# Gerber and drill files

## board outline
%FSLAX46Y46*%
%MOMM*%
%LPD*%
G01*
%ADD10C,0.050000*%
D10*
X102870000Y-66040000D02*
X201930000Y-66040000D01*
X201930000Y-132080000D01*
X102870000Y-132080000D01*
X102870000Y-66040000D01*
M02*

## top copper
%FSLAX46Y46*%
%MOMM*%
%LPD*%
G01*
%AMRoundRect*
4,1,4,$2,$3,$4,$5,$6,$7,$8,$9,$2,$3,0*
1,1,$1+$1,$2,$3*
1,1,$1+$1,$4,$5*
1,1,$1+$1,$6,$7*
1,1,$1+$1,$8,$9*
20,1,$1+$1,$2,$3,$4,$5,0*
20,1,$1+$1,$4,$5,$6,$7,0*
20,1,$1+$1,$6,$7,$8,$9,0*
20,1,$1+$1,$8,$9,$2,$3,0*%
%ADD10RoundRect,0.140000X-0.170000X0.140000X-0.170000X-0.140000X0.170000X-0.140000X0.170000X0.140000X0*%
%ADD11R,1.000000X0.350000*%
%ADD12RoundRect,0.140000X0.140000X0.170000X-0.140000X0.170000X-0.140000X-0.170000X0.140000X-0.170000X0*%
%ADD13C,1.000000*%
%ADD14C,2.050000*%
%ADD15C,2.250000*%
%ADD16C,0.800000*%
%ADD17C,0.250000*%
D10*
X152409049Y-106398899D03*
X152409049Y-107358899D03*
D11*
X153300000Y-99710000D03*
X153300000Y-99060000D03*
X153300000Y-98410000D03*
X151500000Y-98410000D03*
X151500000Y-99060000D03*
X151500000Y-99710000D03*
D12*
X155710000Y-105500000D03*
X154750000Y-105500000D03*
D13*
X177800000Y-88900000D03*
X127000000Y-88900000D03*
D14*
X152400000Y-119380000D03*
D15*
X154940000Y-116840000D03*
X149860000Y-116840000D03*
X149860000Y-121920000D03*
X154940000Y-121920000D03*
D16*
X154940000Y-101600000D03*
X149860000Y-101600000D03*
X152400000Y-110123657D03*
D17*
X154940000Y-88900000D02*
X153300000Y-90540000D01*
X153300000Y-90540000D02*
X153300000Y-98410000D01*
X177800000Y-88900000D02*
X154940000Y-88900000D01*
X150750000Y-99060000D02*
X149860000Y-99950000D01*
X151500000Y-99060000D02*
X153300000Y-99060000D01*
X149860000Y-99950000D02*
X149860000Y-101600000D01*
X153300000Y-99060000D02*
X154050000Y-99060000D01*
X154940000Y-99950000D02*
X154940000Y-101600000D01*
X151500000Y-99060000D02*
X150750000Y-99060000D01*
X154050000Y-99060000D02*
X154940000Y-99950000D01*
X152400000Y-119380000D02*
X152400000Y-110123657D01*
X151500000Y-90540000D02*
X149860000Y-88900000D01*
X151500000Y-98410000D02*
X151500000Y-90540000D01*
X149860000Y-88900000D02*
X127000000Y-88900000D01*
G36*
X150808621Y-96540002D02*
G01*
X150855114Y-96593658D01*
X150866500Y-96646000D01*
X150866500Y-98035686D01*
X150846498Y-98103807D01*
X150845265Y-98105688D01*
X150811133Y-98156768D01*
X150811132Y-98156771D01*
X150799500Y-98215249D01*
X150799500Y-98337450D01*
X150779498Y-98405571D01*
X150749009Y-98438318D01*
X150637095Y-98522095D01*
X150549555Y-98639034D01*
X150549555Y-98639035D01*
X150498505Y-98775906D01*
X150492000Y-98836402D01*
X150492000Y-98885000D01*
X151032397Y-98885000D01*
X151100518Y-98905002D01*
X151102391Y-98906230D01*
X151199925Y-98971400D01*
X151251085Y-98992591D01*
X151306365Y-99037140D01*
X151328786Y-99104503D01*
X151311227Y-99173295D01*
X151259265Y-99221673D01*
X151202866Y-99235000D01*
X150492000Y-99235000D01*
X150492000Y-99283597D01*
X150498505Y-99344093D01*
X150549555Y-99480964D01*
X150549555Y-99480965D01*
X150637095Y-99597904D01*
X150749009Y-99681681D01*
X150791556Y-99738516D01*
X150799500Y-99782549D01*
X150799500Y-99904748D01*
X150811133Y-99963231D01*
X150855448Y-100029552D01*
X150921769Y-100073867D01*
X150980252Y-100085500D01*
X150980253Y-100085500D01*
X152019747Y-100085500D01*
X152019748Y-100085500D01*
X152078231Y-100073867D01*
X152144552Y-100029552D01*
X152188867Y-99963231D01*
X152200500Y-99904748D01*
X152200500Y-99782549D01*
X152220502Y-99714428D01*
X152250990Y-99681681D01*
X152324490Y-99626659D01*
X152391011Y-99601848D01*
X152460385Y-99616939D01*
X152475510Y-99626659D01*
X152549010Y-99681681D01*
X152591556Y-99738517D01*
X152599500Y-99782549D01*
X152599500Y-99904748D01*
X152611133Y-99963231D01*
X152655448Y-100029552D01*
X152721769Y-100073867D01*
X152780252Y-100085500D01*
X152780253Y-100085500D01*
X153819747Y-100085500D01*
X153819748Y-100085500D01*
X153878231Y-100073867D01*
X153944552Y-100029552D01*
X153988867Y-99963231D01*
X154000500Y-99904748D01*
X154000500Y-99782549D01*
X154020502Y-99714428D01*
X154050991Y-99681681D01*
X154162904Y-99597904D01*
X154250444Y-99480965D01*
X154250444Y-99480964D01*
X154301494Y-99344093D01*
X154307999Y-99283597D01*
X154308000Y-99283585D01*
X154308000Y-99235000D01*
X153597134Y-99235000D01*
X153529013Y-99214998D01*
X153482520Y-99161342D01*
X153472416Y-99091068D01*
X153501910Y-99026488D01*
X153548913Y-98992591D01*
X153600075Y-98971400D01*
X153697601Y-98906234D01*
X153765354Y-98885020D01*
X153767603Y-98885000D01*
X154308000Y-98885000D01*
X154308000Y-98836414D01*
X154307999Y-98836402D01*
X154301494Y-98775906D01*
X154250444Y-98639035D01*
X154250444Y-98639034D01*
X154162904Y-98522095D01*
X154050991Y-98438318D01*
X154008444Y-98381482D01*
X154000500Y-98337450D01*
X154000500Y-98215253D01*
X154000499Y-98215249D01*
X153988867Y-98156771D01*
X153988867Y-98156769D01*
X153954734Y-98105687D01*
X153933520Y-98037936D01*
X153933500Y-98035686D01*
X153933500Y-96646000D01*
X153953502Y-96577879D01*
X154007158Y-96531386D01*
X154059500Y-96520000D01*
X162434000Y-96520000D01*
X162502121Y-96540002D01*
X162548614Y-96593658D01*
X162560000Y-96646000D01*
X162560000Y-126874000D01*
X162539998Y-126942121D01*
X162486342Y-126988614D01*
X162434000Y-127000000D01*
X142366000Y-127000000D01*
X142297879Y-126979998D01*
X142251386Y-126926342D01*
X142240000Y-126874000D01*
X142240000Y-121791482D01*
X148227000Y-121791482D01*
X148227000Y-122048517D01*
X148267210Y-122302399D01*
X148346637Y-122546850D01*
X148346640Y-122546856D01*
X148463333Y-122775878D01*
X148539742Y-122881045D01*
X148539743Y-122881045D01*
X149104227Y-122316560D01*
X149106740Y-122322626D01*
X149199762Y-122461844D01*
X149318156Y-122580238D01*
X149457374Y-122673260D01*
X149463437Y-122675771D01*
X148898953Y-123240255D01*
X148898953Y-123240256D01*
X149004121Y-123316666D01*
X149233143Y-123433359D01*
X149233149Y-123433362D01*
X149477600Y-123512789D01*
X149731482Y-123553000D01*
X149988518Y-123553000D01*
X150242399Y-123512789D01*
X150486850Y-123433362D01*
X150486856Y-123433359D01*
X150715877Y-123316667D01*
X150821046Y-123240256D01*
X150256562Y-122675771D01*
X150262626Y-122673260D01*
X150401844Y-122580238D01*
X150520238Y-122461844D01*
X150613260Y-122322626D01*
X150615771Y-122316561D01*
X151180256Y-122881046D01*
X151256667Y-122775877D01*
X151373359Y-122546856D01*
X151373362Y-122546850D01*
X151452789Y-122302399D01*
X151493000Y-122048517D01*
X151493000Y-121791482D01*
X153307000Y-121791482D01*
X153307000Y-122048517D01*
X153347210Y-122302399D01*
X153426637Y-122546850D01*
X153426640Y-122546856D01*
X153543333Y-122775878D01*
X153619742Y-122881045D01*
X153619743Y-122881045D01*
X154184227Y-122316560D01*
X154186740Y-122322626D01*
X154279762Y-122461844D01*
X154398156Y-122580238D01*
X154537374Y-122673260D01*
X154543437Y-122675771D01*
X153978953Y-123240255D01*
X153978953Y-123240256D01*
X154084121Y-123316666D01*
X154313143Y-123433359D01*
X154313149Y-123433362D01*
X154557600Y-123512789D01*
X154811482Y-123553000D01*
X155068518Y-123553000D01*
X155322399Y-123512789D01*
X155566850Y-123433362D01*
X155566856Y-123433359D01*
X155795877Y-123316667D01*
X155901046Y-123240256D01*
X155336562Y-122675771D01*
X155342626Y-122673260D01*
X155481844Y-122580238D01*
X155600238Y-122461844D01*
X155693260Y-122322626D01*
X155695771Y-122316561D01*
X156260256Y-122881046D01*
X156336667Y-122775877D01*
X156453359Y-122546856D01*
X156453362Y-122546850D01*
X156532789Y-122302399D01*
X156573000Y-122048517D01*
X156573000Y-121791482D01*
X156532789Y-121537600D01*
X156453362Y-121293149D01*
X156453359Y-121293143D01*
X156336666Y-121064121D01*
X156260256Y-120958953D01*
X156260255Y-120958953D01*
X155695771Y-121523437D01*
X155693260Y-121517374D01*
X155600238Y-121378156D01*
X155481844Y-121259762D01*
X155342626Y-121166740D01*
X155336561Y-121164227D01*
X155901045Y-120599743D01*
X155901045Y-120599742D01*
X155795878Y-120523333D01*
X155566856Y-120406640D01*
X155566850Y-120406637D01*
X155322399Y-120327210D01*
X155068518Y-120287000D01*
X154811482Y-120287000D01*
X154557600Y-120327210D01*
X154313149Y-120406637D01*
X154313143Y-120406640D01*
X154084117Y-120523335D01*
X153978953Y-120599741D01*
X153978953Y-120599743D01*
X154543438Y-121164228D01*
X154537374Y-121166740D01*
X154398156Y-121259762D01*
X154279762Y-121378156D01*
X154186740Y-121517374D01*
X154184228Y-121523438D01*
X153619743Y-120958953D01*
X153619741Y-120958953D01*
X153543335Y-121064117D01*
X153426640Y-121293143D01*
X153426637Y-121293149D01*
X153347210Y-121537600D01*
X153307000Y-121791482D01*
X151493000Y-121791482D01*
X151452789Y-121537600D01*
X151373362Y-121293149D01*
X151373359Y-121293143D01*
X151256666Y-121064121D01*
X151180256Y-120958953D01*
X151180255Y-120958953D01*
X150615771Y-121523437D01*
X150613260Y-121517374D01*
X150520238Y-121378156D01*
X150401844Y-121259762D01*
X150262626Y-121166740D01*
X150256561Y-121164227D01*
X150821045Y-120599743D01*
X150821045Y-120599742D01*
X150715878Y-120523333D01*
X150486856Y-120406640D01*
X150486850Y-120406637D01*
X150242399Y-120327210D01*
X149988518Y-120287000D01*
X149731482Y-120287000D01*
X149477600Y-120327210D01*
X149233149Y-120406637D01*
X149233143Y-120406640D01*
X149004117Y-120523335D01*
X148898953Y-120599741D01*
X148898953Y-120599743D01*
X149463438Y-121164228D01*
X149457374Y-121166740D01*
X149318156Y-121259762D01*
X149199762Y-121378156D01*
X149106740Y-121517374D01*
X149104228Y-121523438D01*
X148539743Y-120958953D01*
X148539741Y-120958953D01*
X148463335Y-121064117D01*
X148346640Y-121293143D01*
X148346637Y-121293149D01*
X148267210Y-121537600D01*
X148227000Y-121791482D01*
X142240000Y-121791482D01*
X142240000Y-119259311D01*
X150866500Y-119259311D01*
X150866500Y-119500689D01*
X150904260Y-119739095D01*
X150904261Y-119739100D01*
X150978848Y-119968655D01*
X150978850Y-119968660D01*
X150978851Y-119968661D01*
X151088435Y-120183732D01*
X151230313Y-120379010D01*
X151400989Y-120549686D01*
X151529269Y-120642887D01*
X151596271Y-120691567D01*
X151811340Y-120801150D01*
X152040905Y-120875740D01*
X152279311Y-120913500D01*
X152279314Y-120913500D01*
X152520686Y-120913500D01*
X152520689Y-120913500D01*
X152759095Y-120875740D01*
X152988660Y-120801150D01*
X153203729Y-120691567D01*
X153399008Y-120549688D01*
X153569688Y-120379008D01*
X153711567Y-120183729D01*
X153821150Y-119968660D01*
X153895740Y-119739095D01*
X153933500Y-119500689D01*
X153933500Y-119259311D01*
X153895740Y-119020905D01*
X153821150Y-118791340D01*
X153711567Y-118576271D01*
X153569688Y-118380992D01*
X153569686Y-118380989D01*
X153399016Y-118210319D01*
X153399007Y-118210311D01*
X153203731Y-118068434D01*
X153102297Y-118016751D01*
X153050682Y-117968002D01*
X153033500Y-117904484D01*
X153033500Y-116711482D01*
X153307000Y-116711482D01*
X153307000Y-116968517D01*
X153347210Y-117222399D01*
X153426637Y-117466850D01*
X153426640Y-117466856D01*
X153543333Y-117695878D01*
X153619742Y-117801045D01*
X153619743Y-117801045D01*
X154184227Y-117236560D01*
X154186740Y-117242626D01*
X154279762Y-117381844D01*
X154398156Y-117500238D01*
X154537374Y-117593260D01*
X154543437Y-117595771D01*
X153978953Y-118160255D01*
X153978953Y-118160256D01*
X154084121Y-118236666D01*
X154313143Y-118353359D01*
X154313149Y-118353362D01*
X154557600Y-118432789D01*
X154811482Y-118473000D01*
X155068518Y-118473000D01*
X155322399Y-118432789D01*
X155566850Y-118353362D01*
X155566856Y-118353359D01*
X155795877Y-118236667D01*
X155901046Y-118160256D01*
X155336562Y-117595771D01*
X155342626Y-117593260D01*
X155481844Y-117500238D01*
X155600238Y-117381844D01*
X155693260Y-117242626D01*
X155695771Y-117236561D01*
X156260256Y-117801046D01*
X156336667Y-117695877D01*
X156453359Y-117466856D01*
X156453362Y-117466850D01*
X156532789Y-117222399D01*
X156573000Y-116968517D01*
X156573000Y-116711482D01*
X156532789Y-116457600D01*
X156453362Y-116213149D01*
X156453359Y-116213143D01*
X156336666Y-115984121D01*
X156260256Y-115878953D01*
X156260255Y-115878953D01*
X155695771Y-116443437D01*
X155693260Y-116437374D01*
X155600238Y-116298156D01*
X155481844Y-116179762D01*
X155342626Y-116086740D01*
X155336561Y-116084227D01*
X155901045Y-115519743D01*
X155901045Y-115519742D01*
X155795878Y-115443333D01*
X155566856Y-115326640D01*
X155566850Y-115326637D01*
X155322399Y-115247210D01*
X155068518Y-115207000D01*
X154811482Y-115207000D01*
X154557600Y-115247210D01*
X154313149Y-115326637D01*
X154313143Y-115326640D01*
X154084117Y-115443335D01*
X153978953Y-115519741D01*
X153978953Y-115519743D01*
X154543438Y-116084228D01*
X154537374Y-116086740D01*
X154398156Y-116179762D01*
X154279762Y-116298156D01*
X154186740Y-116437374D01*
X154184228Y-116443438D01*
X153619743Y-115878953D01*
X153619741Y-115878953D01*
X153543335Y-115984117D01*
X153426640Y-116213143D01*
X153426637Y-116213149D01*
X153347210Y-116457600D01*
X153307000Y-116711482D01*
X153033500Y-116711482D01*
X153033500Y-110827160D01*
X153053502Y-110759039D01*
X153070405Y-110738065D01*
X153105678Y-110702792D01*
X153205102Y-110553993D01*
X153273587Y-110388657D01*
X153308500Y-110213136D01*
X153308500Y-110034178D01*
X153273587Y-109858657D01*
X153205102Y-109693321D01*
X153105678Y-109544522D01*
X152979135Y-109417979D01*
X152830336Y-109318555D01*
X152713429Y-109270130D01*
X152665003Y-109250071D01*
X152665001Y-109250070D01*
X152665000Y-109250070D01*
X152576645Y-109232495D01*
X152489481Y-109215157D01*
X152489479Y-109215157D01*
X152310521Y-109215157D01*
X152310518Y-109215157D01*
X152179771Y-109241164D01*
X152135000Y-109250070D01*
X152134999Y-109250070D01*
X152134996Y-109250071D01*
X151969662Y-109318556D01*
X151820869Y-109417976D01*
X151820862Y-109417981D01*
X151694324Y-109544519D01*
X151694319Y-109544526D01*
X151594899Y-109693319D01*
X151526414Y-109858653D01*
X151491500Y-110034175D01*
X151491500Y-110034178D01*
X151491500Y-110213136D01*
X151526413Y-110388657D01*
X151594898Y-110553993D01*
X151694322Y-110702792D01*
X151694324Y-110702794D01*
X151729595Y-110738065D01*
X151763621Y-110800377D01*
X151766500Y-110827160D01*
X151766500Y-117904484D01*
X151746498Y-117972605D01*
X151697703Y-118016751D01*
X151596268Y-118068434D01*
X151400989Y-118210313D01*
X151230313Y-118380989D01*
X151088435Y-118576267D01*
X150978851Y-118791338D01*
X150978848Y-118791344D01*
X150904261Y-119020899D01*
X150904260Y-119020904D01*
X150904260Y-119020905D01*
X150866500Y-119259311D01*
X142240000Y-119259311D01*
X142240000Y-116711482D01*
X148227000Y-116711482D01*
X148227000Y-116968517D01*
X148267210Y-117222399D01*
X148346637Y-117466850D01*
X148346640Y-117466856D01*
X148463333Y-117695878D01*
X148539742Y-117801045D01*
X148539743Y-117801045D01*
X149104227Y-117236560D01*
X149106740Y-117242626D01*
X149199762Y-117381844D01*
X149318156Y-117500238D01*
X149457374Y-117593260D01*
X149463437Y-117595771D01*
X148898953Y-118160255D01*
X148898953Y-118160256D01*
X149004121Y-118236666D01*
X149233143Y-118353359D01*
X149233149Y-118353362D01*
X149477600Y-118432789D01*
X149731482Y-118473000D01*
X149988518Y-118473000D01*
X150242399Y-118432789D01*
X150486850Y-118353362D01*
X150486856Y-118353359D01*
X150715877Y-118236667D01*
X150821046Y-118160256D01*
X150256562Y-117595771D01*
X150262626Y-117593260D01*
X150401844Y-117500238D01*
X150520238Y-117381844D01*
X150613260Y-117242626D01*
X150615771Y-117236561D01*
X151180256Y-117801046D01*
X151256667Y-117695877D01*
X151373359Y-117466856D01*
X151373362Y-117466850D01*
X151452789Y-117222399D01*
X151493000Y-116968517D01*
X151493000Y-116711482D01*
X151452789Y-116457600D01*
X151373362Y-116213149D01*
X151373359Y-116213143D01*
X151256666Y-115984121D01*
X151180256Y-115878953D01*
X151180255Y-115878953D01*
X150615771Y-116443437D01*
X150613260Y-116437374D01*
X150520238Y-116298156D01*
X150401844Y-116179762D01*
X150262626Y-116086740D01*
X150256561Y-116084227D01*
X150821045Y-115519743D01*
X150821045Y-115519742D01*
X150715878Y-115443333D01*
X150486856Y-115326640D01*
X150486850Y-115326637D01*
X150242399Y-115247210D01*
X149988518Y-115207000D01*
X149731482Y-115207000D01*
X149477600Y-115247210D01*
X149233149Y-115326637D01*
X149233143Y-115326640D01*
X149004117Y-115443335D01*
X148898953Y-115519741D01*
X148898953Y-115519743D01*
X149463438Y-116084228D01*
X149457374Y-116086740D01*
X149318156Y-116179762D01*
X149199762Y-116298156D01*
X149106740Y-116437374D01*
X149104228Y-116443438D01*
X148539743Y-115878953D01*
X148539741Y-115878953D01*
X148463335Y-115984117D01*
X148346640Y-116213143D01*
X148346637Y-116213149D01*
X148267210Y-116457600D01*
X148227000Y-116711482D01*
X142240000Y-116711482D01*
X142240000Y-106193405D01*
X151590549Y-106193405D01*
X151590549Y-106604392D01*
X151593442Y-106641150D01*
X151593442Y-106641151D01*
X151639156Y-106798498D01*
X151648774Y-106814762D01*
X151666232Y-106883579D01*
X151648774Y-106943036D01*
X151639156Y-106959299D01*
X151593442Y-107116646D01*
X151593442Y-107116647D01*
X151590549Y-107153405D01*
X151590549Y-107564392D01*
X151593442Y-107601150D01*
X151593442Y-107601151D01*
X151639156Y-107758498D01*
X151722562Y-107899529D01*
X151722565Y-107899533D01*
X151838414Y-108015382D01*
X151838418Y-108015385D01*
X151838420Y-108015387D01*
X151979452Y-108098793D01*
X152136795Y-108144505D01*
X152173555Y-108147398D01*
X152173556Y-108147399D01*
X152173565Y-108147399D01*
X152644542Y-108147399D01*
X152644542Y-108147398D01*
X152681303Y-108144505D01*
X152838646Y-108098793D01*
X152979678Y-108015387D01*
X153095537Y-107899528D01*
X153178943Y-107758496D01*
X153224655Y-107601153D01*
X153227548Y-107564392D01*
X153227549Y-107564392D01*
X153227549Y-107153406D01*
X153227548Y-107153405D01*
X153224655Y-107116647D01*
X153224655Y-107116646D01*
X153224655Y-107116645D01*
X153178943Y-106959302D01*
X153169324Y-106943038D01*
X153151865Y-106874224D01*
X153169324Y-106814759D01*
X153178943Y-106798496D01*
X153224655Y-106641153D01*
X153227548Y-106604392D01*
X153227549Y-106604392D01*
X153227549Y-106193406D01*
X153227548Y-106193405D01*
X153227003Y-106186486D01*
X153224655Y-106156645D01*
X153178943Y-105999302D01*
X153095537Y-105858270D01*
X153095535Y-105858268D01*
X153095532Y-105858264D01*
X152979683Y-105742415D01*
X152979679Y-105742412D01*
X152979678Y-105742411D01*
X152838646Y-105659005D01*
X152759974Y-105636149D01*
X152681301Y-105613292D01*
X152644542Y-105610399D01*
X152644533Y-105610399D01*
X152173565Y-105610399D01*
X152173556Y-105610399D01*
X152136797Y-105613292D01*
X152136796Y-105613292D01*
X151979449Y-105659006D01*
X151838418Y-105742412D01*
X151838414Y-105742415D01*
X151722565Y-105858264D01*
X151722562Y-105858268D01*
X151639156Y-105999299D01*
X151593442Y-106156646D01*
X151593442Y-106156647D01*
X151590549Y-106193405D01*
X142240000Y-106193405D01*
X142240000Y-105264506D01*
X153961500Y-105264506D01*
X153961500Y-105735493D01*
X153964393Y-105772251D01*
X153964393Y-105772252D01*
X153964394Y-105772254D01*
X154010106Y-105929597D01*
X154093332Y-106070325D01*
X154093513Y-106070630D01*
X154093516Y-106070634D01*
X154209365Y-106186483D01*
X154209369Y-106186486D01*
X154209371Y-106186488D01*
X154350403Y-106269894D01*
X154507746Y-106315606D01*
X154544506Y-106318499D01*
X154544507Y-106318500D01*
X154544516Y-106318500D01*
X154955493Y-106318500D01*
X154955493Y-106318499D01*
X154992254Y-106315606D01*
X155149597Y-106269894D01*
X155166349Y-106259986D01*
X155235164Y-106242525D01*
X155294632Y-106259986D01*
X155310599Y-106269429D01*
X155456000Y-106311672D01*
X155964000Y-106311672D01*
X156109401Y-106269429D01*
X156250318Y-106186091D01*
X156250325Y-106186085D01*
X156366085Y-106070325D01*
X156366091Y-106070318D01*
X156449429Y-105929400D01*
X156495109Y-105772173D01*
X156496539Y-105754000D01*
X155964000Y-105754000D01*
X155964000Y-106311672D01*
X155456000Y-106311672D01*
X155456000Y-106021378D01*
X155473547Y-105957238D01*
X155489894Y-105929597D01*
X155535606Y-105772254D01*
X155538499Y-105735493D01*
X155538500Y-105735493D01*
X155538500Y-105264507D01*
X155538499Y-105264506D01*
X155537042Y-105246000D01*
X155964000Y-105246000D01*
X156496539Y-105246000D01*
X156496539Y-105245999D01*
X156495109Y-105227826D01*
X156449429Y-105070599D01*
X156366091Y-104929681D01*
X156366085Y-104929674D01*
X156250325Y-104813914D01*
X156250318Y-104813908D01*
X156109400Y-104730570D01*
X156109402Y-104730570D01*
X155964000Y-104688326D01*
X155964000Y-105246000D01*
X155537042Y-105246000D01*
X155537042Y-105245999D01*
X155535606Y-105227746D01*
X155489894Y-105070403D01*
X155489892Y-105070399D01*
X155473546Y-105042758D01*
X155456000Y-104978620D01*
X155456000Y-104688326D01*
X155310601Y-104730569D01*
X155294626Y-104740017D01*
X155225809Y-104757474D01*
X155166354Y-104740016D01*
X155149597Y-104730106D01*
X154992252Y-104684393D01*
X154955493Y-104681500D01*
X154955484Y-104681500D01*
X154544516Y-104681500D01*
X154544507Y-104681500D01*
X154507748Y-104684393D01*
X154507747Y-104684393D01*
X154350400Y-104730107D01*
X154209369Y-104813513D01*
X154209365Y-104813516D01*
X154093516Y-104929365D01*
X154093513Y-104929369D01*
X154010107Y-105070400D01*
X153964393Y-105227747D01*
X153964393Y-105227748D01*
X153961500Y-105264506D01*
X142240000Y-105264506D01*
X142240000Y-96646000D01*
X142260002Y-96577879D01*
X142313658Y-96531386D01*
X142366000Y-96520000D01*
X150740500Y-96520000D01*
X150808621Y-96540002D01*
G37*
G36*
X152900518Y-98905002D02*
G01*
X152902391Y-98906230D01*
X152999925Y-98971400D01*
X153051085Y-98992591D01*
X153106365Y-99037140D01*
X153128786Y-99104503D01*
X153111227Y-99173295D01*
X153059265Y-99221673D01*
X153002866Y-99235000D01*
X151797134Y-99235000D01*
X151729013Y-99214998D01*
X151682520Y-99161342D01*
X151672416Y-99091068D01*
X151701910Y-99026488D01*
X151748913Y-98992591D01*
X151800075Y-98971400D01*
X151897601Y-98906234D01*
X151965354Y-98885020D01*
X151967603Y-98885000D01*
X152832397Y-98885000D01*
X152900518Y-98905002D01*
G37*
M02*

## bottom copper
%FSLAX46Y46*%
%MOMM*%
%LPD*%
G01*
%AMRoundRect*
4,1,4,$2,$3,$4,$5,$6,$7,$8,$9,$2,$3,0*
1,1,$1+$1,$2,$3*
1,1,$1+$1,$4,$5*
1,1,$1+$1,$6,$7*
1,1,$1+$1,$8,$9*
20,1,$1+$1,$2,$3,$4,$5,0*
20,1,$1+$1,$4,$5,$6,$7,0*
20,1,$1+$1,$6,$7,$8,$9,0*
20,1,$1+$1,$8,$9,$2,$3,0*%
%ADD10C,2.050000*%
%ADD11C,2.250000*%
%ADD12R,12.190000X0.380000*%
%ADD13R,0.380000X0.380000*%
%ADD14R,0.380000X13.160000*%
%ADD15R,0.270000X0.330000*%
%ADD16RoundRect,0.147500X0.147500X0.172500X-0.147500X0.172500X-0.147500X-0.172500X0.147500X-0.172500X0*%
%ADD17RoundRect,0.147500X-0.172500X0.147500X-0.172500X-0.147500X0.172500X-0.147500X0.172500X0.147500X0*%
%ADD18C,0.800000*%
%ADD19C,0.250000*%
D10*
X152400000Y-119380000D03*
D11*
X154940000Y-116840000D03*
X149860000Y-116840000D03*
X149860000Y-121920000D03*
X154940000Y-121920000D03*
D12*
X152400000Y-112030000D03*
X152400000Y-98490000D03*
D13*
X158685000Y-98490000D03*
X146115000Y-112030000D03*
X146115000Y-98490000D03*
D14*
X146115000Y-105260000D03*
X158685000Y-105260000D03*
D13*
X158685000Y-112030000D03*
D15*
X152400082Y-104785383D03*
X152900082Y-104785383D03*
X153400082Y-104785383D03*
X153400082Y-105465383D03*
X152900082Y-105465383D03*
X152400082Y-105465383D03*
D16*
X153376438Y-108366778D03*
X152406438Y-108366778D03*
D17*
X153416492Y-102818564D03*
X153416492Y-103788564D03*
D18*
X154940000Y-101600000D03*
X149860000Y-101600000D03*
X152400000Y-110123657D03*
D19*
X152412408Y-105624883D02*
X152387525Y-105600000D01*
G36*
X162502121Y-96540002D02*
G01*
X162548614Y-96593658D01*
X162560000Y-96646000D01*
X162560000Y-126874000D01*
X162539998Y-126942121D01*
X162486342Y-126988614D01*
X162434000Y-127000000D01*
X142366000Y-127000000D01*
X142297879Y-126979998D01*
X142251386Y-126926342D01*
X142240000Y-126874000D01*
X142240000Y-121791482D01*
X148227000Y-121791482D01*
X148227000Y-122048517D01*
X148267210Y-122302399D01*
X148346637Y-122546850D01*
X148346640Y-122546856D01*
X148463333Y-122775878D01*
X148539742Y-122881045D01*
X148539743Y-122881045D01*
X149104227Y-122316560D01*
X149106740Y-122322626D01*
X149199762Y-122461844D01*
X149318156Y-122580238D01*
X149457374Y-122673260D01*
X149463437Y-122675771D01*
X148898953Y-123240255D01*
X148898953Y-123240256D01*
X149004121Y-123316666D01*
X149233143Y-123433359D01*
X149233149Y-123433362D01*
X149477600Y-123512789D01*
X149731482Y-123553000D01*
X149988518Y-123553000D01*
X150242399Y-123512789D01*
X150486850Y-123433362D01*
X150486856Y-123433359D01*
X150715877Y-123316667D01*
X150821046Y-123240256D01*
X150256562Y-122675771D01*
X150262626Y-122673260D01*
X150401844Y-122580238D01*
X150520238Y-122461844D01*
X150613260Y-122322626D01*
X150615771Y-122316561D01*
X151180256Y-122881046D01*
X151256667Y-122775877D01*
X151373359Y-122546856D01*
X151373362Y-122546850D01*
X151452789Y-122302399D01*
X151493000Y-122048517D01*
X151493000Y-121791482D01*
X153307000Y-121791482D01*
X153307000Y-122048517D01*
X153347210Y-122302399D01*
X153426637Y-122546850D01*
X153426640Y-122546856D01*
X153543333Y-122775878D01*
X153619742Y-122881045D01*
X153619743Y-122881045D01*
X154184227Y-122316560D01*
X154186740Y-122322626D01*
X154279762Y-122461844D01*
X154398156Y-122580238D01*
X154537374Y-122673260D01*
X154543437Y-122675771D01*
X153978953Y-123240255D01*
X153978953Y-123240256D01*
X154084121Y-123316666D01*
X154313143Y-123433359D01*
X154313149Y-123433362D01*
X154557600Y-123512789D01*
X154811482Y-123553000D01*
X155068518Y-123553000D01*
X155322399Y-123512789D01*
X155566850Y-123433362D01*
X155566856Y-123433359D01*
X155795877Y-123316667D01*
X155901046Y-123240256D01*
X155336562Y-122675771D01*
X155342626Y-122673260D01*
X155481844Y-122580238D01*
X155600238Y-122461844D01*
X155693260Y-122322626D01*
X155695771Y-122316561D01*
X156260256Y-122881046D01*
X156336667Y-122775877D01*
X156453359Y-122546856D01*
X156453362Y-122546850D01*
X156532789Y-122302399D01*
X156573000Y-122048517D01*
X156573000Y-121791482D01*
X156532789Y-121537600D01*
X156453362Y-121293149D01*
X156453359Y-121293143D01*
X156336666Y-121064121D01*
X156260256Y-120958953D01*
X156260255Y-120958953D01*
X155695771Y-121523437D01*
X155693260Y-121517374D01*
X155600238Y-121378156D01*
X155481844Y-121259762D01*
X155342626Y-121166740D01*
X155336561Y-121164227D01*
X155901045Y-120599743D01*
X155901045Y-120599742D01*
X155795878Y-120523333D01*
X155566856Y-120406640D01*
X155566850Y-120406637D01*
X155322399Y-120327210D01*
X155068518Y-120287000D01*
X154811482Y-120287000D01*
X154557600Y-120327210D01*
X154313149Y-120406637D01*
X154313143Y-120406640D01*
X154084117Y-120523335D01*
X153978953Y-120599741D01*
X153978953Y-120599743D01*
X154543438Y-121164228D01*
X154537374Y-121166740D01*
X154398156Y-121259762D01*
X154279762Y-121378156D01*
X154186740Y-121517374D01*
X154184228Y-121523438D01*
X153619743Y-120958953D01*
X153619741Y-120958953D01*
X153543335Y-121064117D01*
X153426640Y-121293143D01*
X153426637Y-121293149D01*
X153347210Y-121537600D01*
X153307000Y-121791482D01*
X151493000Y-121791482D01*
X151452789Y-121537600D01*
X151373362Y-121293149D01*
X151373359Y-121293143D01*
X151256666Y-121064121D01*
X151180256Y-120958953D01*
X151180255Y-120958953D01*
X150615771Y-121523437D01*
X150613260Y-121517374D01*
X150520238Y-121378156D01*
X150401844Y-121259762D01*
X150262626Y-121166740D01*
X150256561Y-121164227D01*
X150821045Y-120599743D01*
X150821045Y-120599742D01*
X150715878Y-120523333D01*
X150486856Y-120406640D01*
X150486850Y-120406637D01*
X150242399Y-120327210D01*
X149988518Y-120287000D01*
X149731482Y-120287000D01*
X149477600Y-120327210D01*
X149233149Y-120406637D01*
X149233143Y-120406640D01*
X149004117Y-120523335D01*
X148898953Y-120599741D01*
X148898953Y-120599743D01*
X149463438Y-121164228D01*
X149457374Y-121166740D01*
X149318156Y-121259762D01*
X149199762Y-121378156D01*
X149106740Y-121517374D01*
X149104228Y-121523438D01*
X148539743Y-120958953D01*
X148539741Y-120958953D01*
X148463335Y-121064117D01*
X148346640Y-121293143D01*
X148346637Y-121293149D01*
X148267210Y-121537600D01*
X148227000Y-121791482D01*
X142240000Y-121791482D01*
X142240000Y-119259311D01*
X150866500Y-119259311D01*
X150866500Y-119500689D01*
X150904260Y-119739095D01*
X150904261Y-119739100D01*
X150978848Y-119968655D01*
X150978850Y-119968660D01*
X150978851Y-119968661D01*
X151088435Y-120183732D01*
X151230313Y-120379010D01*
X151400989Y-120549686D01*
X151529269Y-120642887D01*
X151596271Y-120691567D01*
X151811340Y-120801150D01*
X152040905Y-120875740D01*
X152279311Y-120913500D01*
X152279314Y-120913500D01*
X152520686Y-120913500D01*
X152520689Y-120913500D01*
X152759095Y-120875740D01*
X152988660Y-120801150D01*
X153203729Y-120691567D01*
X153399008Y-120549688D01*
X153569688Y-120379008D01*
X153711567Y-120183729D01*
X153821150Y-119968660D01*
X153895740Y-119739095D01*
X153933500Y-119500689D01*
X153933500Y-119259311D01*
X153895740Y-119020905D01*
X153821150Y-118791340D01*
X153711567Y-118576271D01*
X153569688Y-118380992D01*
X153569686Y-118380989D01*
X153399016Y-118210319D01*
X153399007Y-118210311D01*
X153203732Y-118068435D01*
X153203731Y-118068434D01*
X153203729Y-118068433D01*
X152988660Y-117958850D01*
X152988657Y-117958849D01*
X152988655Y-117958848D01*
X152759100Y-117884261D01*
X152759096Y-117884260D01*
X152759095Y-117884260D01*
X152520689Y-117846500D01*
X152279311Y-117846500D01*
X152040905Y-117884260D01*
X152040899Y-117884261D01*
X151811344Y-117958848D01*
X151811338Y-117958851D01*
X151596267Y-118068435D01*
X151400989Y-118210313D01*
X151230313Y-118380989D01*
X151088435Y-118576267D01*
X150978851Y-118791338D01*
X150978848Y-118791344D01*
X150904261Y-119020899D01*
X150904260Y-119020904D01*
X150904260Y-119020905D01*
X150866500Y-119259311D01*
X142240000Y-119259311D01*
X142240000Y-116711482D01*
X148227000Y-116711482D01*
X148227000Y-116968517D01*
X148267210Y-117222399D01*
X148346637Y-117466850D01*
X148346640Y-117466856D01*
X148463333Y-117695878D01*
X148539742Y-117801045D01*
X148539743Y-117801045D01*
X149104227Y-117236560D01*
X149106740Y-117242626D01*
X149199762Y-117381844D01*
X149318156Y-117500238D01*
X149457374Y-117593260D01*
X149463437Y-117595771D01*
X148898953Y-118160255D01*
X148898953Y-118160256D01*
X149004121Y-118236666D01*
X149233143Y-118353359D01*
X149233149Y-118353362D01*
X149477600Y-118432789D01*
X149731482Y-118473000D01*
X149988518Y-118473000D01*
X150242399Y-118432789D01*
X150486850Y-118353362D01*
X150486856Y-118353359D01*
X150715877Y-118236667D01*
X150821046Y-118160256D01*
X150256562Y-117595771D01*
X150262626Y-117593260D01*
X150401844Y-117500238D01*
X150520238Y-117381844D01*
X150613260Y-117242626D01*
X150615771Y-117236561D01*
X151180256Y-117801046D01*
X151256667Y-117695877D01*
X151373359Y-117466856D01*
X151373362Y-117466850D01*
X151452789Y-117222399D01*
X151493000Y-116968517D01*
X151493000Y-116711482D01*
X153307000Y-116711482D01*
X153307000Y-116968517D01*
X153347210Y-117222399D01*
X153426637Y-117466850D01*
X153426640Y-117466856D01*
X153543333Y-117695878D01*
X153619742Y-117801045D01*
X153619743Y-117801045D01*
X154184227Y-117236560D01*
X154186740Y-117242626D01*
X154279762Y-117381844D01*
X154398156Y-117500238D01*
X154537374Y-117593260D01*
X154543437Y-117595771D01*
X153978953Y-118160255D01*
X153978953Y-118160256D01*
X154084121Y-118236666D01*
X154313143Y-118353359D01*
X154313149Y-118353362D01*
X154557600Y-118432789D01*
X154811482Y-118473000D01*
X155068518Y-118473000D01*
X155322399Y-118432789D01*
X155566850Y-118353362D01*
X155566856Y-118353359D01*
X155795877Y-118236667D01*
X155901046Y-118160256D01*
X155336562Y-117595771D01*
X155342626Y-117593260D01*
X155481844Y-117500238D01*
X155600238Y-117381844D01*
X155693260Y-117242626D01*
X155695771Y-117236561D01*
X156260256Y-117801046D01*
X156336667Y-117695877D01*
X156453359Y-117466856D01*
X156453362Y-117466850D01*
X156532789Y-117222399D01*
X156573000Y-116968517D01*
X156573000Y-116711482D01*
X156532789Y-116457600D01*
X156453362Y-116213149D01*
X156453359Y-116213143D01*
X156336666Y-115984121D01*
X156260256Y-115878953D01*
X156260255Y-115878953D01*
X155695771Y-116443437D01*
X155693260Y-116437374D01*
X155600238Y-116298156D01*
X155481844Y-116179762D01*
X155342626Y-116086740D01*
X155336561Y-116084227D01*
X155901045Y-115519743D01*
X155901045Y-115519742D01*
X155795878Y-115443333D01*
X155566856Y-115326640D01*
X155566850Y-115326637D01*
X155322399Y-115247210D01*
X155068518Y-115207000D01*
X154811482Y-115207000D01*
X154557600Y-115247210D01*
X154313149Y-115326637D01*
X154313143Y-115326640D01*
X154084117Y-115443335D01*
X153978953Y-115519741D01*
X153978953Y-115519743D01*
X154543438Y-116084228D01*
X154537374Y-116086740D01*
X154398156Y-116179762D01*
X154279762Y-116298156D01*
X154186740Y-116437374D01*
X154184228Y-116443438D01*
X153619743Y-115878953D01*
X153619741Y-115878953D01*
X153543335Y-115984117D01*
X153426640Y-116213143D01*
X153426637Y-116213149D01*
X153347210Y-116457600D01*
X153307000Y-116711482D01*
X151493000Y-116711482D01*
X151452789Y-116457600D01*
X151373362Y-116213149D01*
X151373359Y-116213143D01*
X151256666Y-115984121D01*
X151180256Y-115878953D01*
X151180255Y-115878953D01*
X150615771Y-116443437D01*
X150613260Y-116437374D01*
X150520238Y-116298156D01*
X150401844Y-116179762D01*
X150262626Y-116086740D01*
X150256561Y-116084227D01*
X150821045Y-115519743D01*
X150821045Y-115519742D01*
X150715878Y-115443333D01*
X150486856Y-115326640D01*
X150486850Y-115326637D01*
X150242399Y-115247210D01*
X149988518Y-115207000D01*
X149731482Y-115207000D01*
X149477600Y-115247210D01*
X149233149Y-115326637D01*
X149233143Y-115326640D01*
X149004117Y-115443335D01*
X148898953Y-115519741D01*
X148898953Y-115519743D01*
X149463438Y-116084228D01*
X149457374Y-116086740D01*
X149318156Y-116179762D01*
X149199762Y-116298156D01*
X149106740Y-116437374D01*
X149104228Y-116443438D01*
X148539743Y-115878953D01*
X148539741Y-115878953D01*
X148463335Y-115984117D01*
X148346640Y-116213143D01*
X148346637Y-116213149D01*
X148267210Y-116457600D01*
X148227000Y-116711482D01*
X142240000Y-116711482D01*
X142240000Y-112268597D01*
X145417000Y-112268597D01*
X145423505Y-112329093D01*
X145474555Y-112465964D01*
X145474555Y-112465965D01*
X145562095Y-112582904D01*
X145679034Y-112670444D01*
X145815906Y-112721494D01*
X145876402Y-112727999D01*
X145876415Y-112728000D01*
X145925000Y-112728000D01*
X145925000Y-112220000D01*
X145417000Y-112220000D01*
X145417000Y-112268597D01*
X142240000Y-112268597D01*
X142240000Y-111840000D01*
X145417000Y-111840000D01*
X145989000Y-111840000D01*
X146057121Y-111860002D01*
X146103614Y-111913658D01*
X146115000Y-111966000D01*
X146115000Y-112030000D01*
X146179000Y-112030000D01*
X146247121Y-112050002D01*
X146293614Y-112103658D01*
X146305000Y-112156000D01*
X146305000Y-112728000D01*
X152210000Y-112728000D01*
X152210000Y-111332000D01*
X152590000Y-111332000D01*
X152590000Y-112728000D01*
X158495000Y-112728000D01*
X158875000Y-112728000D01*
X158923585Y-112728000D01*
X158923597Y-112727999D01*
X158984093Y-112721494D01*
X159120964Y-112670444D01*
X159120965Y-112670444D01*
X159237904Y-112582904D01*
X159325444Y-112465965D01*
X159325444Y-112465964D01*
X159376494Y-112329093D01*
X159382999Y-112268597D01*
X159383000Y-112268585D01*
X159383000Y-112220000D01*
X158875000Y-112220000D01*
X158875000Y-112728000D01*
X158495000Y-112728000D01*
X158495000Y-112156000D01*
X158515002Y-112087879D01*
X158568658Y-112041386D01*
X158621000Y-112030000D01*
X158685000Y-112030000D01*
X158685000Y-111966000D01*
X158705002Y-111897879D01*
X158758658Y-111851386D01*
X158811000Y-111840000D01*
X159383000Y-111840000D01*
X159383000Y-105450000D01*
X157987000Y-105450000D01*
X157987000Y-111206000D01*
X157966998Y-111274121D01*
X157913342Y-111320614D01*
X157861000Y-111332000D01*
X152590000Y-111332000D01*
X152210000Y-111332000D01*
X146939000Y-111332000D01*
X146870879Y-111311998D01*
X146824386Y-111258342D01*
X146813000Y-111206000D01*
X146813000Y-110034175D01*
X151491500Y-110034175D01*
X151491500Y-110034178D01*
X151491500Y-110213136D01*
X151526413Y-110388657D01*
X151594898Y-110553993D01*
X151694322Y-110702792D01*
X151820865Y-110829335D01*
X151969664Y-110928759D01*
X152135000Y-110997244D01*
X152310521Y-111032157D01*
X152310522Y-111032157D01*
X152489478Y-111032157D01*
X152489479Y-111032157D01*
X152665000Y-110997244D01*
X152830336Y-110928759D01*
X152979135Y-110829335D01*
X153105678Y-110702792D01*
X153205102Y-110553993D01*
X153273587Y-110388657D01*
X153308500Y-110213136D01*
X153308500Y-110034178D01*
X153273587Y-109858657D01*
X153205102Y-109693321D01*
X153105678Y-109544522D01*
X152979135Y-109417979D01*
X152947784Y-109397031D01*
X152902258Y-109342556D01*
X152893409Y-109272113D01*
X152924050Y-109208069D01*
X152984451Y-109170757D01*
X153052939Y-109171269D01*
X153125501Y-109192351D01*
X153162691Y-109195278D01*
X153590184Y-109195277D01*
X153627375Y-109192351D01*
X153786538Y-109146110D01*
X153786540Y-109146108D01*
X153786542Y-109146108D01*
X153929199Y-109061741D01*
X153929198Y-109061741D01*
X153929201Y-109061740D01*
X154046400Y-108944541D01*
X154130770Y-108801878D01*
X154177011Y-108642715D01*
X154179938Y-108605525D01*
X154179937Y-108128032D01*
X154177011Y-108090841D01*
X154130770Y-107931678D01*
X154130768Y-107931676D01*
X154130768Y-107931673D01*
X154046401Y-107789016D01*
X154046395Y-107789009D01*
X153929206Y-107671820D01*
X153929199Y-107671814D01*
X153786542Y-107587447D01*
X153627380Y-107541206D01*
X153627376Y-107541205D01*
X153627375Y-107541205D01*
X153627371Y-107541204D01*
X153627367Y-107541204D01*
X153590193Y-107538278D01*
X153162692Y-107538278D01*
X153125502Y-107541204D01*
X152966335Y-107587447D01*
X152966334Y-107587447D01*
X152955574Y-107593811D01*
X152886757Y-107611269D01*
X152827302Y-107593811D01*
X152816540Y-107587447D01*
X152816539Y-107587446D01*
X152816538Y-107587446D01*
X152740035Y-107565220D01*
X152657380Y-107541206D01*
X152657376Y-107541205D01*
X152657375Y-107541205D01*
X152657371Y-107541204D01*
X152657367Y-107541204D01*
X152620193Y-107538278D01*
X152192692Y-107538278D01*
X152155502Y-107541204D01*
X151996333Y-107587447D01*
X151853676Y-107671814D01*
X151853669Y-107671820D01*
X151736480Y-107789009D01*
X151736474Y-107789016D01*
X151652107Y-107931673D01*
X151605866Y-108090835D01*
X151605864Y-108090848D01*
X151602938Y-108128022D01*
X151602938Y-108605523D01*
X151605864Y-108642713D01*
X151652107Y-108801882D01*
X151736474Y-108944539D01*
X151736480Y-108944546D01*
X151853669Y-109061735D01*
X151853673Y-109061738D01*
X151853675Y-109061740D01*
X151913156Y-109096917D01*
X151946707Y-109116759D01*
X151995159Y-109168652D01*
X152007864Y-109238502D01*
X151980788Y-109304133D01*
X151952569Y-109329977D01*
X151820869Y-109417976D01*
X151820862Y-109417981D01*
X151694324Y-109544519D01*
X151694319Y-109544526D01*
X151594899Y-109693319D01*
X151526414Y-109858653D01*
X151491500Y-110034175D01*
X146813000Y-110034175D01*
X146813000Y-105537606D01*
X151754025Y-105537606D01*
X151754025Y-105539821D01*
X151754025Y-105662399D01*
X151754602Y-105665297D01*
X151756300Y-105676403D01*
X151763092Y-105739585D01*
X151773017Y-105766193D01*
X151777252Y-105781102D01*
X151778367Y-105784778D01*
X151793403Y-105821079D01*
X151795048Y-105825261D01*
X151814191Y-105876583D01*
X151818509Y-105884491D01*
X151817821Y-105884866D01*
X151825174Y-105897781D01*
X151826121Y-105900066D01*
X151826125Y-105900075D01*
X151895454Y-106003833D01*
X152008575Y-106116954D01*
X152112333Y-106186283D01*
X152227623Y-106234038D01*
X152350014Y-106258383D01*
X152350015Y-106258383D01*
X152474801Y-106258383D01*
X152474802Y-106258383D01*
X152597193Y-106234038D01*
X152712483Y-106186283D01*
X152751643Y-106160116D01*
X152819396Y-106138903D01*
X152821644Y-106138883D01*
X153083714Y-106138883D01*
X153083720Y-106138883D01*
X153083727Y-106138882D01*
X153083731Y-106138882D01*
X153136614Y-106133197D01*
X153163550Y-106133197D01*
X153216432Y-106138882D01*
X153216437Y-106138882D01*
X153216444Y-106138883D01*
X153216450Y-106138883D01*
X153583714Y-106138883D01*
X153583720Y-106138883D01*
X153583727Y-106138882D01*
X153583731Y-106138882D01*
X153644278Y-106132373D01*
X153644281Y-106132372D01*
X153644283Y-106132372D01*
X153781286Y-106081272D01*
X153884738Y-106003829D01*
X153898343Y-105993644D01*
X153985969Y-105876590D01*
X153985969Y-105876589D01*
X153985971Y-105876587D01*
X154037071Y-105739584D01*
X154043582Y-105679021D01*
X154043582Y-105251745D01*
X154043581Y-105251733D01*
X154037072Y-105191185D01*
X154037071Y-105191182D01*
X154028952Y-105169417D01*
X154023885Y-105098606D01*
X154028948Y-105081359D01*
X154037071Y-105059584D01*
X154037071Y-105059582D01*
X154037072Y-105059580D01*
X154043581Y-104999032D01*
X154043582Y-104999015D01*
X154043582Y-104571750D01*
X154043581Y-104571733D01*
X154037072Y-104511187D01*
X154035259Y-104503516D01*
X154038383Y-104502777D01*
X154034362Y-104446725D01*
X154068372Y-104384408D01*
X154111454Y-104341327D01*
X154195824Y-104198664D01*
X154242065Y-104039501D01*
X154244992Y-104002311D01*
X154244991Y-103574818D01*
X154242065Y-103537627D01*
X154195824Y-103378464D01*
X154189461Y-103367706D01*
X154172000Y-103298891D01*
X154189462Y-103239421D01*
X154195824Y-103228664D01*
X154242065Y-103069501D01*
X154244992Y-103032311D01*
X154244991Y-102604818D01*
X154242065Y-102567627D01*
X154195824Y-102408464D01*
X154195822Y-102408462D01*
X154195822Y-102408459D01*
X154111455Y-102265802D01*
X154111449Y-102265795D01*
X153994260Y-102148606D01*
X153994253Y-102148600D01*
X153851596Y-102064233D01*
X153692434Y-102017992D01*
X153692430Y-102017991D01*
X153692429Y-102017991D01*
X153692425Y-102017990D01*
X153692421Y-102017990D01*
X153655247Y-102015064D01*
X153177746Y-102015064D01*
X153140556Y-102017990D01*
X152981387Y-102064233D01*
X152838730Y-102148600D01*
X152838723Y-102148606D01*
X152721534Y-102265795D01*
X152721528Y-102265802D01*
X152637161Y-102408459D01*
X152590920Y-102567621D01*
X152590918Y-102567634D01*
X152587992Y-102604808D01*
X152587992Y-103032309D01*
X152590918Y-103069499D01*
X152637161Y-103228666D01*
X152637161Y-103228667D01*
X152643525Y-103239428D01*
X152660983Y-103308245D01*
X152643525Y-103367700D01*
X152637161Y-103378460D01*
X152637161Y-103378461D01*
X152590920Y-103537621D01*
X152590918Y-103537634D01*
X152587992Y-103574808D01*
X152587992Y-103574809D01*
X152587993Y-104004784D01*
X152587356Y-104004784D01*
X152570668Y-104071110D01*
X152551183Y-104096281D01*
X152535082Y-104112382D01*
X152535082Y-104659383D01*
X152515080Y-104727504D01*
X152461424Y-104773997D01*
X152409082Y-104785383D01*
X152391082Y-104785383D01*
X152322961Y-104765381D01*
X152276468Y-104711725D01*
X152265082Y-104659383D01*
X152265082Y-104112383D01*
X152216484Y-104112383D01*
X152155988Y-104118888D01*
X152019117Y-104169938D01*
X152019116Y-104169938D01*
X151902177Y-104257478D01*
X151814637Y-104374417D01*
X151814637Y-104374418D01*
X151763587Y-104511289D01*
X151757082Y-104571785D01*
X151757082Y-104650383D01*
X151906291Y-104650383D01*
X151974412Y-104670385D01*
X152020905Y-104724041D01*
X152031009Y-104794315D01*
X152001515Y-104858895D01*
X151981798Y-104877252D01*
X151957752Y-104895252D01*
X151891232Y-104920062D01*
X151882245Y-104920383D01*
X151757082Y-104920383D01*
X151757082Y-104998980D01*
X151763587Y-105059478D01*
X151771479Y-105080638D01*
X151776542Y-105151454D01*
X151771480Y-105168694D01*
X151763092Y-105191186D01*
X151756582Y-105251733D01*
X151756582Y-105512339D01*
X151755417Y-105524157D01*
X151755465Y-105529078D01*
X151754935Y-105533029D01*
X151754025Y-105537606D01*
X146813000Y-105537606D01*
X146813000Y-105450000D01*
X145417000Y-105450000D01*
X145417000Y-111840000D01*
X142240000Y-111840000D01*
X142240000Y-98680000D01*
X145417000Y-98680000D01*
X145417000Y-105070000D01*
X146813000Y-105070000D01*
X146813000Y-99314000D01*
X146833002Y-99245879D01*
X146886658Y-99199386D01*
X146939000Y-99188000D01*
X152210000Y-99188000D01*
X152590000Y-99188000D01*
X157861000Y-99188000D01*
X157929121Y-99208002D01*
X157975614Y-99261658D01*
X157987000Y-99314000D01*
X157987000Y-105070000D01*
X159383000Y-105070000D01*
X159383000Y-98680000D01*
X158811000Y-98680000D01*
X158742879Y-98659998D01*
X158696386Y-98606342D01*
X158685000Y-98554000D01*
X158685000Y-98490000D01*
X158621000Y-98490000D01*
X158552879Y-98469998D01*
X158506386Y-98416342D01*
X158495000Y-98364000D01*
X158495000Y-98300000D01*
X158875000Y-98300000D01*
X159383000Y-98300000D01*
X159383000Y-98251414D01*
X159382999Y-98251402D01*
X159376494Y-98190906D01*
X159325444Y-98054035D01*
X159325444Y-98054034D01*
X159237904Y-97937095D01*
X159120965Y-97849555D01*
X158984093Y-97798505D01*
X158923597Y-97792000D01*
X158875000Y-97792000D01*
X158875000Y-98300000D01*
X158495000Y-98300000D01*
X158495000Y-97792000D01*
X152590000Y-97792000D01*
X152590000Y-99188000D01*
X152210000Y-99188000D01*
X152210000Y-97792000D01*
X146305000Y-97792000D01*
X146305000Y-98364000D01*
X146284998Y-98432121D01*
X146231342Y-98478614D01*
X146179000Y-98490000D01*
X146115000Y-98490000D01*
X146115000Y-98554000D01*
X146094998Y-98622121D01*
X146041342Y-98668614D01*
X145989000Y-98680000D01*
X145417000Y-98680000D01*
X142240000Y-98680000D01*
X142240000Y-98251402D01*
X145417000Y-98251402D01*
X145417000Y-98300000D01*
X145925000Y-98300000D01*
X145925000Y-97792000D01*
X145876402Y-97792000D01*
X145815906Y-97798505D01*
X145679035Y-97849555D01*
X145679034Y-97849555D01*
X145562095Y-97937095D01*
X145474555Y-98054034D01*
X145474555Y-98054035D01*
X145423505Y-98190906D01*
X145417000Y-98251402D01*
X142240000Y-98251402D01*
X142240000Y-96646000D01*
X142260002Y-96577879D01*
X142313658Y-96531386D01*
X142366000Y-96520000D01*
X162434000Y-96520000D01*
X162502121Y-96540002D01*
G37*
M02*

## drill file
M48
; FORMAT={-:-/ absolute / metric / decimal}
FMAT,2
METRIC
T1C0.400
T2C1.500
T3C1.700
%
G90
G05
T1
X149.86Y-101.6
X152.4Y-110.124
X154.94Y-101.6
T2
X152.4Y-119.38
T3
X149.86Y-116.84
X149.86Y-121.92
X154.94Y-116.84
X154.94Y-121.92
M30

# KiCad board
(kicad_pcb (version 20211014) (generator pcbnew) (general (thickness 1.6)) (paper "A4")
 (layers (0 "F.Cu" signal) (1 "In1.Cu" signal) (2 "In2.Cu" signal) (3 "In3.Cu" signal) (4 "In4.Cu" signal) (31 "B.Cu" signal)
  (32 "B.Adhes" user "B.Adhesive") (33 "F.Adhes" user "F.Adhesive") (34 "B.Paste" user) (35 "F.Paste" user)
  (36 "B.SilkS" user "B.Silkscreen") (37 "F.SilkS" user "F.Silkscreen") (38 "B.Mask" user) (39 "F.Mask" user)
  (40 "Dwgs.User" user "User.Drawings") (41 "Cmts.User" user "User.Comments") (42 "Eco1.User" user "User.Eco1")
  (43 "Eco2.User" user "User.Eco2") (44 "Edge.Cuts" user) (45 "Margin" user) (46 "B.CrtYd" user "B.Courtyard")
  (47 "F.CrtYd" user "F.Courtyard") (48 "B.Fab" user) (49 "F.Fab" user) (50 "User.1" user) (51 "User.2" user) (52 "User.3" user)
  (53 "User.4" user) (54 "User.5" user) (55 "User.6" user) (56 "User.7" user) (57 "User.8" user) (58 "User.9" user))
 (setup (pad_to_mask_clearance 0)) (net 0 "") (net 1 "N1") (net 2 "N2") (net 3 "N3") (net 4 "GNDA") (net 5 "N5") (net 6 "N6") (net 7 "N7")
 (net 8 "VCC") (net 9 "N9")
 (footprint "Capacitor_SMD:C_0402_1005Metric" (layer "F.Cu") (at 152.409049 106.878899 -90)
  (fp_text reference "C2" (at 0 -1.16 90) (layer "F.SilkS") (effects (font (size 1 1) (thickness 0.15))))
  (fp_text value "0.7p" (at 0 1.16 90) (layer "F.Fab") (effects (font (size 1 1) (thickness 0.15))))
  (pad "1" smd roundrect (at -0.48 0 270) (size 0.56 0.62) (layers "F.Cu" "F.Paste" "F.Mask") (roundrect_rratio 0.25) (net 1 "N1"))
  (pad "2" smd roundrect (at 0.48 0 270) (size 0.56 0.62) (layers "F.Cu" "F.Paste" "F.Mask") (roundrect_rratio 0.25) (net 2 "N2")))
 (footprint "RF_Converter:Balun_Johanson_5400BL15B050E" (layer "F.Cu") (at 152.4 99.06 180)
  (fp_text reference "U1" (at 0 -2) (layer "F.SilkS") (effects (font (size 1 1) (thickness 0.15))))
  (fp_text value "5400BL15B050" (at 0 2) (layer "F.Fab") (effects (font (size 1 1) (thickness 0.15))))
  (pad "1" smd rect (at -0.9 -0.65 180) (size 1 0.35) (layers "F.Cu" "F.Paste" "F.Mask") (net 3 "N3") (clearance 0.2))
  (pad "2" smd rect (at -0.9 0 180) (size 1 0.35) (layers "F.Cu" "F.Paste" "F.Mask") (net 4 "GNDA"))
  (pad "3" smd rect (at -0.9 0.65 180) (size 1 0.35) (layers "F.Cu" "F.Paste" "F.Mask") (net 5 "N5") (clearance 0.2))
  (pad "4" smd rect (at 0.9 0.65 180) (size 1 0.35) (layers "F.Cu" "F.Paste" "F.Mask") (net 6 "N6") (clearance 0.2))
  (pad "5" smd rect (at 0.9 0 180) (size 1 0.35) (layers "F.Cu" "F.Paste" "F.Mask") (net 4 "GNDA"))
  (pad "6" smd rect (at 0.9 -0.65 180) (size 1 0.35) (layers "F.Cu" "F.Paste" "F.Mask") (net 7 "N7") (clearance 0.2)))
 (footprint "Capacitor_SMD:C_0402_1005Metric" (layer "F.Cu") (at 155.23 105.5 180)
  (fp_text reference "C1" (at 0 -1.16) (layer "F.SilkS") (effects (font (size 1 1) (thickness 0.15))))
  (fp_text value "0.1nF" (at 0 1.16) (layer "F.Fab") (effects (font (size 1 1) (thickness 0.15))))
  (pad "1" smd roundrect (at -0.48 0 180) (size 0.56 0.62) (layers "F.Cu" "F.Paste" "F.Mask") (roundrect_rratio 0.25) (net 4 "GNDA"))
  (pad "2" smd roundrect (at 0.48 0 180) (size 0.56 0.62) (layers "F.Cu" "F.Paste" "F.Mask") (roundrect_rratio 0.25) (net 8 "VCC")))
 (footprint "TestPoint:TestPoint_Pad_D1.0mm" (layer "F.Cu") (at 177.8 88.9)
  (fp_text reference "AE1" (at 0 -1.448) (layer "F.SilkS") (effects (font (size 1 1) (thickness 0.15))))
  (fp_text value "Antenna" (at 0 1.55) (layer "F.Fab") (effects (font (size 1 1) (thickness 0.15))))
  (pad "1" smd circle (at 0 0) (size 1 1) (layers "F.Cu" "F.Mask") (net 5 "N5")))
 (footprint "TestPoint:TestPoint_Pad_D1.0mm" (layer "F.Cu") (at 127 88.9 90)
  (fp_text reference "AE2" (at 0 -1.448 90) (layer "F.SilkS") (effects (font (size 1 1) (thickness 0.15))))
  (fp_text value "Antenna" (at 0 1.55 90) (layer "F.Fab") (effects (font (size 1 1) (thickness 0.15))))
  (pad "1" smd circle (at 0 0 90) (size 1 1) (layers "F.Cu" "F.Mask") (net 6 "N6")))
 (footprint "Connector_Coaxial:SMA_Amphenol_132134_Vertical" (layer "B.Cu") (at 152.4 119.38 180)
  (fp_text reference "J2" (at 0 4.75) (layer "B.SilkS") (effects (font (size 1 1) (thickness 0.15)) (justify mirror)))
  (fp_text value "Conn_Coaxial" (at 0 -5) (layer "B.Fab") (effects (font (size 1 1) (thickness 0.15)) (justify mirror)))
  (pad "1" thru_hole circle (at 0 0 180) (size 2.05 2.05) (drill 1.5) (layers *.Cu *.Mask) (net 2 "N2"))
  (pad "2" thru_hole circle (at -2.54 2.54 180) (size 2.25 2.25) (drill 1.7) (layers *.Cu *.Mask) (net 4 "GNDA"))
  (pad "2" thru_hole circle (at 2.54 2.54 180) (size 2.25 2.25) (drill 1.7) (layers *.Cu *.Mask) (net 4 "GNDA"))
  (pad "2" thru_hole circle (at 2.54 -2.54 180) (size 2.25 2.25) (drill 1.7) (layers *.Cu *.Mask) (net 4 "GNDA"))
  (pad "2" thru_hole circle (at -2.54 -2.54 180) (size 2.25 2.25) (drill 1.7) (layers *.Cu *.Mask) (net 4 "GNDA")))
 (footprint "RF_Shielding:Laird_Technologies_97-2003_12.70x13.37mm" (layer "B.Cu") (at 152.4 105.26 180)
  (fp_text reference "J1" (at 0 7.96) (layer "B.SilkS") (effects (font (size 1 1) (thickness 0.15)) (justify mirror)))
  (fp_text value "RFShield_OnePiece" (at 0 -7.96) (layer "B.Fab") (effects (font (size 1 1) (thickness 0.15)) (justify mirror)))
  (pad "1" smd rect (at 0 -6.77 180) (size 12.19 0.38) (layers "B.Cu" "B.Paste" "B.Mask") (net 4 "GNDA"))
  (pad "1" smd rect (at 0 6.77 180) (size 12.19 0.38) (layers "B.Cu" "B.Paste" "B.Mask") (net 4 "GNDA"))
  (pad "1" smd rect (at -6.285 6.77 180) (size 0.38 0.38) (layers "B.Cu" "B.Paste" "B.Mask") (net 4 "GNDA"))
  (pad "1" smd rect (at 6.285 -6.77 180) (size 0.38 0.38) (layers "B.Cu" "B.Paste" "B.Mask") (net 4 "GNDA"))
  (pad "1" smd rect (at 6.285 6.77 180) (size 0.38 0.38) (layers "B.Cu" "B.Paste" "B.Mask") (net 4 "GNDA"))
  (pad "1" smd rect (at 6.285 0 180) (size 0.38 13.16) (layers "B.Cu" "B.Paste" "B.Mask") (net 4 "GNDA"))
  (pad "1" smd rect (at -6.285 0 180) (size 0.38 13.16) (layers "B.Cu" "B.Paste" "B.Mask") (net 4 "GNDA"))
  (pad "1" smd rect (at -6.285 -6.77 180) (size 0.38 0.38) (layers "B.Cu" "B.Paste" "B.Mask") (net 4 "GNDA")))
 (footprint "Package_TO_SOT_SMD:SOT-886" (layer "B.Cu") (at 152.900082 105.125383 -90)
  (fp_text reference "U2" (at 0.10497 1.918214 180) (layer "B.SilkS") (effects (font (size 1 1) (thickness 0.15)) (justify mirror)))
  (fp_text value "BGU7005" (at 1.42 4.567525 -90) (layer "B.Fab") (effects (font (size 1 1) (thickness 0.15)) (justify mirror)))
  (pad "1" smd rect (at -0.34 0.5 270) (size 0.33 0.27) (layers "B.Cu" "B.Paste" "B.Mask") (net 4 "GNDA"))
  (pad "2" smd rect (at -0.34 0 270) (size 0.33 0.27) (layers "B.Cu" "B.Paste" "B.Mask") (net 4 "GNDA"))
  (pad "3" smd rect (at -0.34 -0.5 270) (size 0.33 0.27) (layers "B.Cu" "B.Paste" "B.Mask") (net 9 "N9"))
  (pad "4" smd rect (at 0.34 -0.5 270) (size 0.33 0.27) (layers "B.Cu" "B.Paste" "B.Mask") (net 8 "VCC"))
  (pad "5" smd rect (at 0.34 0 270) (size 0.33 0.27) (layers "B.Cu" "B.Paste" "B.Mask") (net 8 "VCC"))
  (pad "6" smd rect (at 0.34 0.5 270) (size 0.33 0.27) (layers "B.Cu" "B.Paste" "B.Mask") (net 1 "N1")))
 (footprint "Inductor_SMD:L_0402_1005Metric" (layer "B.Cu") (at 152.891438 108.366778 180)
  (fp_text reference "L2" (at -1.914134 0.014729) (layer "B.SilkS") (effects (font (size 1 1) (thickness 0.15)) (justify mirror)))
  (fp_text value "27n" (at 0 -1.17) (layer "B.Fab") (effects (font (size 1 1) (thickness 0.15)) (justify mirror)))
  (pad "1" smd roundrect (at -0.485 0 180) (size 0.59 0.64) (layers "B.Cu" "B.Paste" "B.Mask") (roundrect_rratio 0.25) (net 8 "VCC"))
  (pad "2" smd roundrect (at 0.485 0 180) (size 0.59 0.64) (layers "B.Cu" "B.Paste" "B.Mask") (roundrect_rratio 0.25) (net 2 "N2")))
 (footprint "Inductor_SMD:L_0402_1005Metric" (layer "B.Cu") (at 153.416492 103.303564 -90)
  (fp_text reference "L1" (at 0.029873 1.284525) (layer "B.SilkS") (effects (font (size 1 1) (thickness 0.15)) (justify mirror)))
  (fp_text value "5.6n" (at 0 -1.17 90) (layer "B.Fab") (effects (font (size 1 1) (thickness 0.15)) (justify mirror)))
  (pad "1" smd roundrect (at -0.485 0 270) (size 0.59 0.64) (layers "B.Cu" "B.Paste" "B.Mask") (roundrect_rratio 0.25) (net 3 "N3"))
  (pad "2" smd roundrect (at 0.485 0 270) (size 0.59 0.64) (layers "B.Cu" "B.Paste" "B.Mask") (roundrect_rratio 0.25) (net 9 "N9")))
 (gr_rect (start 102.87 66.04) (end 201.93 132.08) (layer "Edge.Cuts") (width 0.05) (fill none))
 (segment (start 154.94 88.9) (end 153.3 90.54) (width 0.25) (layer "F.Cu") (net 5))
 (segment (start 153.3 90.54) (end 153.3 98.41) (width 0.25) (layer "F.Cu") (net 5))
 (segment (start 177.8 88.9) (end 154.94 88.9) (width 0.25) (layer "F.Cu") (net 5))
 (segment (start 150.75 99.06) (end 149.86 99.95) (width 0.25) (layer "F.Cu") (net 4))
 (segment (start 151.5 99.06) (end 153.3 99.06) (width 0.25) (layer "F.Cu") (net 4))
 (segment (start 149.86 99.95) (end 149.86 101.6) (width 0.25) (layer "F.Cu") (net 4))
 (segment (start 153.3 99.06) (end 154.05 99.06) (width 0.25) (layer "F.Cu") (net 4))
 (segment (start 154.94 99.95) (end 154.94 101.6) (width 0.25) (layer "F.Cu") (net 4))
 (segment (start 151.5 99.06) (end 150.75 99.06) (width 0.25) (layer "F.Cu") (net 4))
 (segment (start 154.05 99.06) (end 154.94 99.95) (width 0.25) (layer "F.Cu") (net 4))
 (via (at 154.94 101.6) (size 0.8) (drill 0.4) (layers "F.Cu" "B.Cu") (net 4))
 (via (at 149.86 101.6) (size 0.8) (drill 0.4) (layers "F.Cu" "B.Cu") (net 4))
 (segment (start 152.412408 105.624883) (end 152.387525 105.6) (width 0.25) (layer "B.Cu") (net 1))
 (segment (start 152.4 119.38) (end 152.4 110.123657) (width 0.25) (layer "F.Cu") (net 2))
 (via (at 152.4 110.123657) (size 0.8) (drill 0.4) (layers "F.Cu" "B.Cu") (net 2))
 (segment (start 151.5 90.54) (end 149.86 88.9) (width 0.25) (layer "F.Cu") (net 6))
 (segment (start 151.5 98.41) (end 151.5 90.54) (width 0.25) (layer "F.Cu") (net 6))
 (segment (start 149.86 88.9) (end 127 88.9) (width 0.25) (layer "F.Cu") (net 6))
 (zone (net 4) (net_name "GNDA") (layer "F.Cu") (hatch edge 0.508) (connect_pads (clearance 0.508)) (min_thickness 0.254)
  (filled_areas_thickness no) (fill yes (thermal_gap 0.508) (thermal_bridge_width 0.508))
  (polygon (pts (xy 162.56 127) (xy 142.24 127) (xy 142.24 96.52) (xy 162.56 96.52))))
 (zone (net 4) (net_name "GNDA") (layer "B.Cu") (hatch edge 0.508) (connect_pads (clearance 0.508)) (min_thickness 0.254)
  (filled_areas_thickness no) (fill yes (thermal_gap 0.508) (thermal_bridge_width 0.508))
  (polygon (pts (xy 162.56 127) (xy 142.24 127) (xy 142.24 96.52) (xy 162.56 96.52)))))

